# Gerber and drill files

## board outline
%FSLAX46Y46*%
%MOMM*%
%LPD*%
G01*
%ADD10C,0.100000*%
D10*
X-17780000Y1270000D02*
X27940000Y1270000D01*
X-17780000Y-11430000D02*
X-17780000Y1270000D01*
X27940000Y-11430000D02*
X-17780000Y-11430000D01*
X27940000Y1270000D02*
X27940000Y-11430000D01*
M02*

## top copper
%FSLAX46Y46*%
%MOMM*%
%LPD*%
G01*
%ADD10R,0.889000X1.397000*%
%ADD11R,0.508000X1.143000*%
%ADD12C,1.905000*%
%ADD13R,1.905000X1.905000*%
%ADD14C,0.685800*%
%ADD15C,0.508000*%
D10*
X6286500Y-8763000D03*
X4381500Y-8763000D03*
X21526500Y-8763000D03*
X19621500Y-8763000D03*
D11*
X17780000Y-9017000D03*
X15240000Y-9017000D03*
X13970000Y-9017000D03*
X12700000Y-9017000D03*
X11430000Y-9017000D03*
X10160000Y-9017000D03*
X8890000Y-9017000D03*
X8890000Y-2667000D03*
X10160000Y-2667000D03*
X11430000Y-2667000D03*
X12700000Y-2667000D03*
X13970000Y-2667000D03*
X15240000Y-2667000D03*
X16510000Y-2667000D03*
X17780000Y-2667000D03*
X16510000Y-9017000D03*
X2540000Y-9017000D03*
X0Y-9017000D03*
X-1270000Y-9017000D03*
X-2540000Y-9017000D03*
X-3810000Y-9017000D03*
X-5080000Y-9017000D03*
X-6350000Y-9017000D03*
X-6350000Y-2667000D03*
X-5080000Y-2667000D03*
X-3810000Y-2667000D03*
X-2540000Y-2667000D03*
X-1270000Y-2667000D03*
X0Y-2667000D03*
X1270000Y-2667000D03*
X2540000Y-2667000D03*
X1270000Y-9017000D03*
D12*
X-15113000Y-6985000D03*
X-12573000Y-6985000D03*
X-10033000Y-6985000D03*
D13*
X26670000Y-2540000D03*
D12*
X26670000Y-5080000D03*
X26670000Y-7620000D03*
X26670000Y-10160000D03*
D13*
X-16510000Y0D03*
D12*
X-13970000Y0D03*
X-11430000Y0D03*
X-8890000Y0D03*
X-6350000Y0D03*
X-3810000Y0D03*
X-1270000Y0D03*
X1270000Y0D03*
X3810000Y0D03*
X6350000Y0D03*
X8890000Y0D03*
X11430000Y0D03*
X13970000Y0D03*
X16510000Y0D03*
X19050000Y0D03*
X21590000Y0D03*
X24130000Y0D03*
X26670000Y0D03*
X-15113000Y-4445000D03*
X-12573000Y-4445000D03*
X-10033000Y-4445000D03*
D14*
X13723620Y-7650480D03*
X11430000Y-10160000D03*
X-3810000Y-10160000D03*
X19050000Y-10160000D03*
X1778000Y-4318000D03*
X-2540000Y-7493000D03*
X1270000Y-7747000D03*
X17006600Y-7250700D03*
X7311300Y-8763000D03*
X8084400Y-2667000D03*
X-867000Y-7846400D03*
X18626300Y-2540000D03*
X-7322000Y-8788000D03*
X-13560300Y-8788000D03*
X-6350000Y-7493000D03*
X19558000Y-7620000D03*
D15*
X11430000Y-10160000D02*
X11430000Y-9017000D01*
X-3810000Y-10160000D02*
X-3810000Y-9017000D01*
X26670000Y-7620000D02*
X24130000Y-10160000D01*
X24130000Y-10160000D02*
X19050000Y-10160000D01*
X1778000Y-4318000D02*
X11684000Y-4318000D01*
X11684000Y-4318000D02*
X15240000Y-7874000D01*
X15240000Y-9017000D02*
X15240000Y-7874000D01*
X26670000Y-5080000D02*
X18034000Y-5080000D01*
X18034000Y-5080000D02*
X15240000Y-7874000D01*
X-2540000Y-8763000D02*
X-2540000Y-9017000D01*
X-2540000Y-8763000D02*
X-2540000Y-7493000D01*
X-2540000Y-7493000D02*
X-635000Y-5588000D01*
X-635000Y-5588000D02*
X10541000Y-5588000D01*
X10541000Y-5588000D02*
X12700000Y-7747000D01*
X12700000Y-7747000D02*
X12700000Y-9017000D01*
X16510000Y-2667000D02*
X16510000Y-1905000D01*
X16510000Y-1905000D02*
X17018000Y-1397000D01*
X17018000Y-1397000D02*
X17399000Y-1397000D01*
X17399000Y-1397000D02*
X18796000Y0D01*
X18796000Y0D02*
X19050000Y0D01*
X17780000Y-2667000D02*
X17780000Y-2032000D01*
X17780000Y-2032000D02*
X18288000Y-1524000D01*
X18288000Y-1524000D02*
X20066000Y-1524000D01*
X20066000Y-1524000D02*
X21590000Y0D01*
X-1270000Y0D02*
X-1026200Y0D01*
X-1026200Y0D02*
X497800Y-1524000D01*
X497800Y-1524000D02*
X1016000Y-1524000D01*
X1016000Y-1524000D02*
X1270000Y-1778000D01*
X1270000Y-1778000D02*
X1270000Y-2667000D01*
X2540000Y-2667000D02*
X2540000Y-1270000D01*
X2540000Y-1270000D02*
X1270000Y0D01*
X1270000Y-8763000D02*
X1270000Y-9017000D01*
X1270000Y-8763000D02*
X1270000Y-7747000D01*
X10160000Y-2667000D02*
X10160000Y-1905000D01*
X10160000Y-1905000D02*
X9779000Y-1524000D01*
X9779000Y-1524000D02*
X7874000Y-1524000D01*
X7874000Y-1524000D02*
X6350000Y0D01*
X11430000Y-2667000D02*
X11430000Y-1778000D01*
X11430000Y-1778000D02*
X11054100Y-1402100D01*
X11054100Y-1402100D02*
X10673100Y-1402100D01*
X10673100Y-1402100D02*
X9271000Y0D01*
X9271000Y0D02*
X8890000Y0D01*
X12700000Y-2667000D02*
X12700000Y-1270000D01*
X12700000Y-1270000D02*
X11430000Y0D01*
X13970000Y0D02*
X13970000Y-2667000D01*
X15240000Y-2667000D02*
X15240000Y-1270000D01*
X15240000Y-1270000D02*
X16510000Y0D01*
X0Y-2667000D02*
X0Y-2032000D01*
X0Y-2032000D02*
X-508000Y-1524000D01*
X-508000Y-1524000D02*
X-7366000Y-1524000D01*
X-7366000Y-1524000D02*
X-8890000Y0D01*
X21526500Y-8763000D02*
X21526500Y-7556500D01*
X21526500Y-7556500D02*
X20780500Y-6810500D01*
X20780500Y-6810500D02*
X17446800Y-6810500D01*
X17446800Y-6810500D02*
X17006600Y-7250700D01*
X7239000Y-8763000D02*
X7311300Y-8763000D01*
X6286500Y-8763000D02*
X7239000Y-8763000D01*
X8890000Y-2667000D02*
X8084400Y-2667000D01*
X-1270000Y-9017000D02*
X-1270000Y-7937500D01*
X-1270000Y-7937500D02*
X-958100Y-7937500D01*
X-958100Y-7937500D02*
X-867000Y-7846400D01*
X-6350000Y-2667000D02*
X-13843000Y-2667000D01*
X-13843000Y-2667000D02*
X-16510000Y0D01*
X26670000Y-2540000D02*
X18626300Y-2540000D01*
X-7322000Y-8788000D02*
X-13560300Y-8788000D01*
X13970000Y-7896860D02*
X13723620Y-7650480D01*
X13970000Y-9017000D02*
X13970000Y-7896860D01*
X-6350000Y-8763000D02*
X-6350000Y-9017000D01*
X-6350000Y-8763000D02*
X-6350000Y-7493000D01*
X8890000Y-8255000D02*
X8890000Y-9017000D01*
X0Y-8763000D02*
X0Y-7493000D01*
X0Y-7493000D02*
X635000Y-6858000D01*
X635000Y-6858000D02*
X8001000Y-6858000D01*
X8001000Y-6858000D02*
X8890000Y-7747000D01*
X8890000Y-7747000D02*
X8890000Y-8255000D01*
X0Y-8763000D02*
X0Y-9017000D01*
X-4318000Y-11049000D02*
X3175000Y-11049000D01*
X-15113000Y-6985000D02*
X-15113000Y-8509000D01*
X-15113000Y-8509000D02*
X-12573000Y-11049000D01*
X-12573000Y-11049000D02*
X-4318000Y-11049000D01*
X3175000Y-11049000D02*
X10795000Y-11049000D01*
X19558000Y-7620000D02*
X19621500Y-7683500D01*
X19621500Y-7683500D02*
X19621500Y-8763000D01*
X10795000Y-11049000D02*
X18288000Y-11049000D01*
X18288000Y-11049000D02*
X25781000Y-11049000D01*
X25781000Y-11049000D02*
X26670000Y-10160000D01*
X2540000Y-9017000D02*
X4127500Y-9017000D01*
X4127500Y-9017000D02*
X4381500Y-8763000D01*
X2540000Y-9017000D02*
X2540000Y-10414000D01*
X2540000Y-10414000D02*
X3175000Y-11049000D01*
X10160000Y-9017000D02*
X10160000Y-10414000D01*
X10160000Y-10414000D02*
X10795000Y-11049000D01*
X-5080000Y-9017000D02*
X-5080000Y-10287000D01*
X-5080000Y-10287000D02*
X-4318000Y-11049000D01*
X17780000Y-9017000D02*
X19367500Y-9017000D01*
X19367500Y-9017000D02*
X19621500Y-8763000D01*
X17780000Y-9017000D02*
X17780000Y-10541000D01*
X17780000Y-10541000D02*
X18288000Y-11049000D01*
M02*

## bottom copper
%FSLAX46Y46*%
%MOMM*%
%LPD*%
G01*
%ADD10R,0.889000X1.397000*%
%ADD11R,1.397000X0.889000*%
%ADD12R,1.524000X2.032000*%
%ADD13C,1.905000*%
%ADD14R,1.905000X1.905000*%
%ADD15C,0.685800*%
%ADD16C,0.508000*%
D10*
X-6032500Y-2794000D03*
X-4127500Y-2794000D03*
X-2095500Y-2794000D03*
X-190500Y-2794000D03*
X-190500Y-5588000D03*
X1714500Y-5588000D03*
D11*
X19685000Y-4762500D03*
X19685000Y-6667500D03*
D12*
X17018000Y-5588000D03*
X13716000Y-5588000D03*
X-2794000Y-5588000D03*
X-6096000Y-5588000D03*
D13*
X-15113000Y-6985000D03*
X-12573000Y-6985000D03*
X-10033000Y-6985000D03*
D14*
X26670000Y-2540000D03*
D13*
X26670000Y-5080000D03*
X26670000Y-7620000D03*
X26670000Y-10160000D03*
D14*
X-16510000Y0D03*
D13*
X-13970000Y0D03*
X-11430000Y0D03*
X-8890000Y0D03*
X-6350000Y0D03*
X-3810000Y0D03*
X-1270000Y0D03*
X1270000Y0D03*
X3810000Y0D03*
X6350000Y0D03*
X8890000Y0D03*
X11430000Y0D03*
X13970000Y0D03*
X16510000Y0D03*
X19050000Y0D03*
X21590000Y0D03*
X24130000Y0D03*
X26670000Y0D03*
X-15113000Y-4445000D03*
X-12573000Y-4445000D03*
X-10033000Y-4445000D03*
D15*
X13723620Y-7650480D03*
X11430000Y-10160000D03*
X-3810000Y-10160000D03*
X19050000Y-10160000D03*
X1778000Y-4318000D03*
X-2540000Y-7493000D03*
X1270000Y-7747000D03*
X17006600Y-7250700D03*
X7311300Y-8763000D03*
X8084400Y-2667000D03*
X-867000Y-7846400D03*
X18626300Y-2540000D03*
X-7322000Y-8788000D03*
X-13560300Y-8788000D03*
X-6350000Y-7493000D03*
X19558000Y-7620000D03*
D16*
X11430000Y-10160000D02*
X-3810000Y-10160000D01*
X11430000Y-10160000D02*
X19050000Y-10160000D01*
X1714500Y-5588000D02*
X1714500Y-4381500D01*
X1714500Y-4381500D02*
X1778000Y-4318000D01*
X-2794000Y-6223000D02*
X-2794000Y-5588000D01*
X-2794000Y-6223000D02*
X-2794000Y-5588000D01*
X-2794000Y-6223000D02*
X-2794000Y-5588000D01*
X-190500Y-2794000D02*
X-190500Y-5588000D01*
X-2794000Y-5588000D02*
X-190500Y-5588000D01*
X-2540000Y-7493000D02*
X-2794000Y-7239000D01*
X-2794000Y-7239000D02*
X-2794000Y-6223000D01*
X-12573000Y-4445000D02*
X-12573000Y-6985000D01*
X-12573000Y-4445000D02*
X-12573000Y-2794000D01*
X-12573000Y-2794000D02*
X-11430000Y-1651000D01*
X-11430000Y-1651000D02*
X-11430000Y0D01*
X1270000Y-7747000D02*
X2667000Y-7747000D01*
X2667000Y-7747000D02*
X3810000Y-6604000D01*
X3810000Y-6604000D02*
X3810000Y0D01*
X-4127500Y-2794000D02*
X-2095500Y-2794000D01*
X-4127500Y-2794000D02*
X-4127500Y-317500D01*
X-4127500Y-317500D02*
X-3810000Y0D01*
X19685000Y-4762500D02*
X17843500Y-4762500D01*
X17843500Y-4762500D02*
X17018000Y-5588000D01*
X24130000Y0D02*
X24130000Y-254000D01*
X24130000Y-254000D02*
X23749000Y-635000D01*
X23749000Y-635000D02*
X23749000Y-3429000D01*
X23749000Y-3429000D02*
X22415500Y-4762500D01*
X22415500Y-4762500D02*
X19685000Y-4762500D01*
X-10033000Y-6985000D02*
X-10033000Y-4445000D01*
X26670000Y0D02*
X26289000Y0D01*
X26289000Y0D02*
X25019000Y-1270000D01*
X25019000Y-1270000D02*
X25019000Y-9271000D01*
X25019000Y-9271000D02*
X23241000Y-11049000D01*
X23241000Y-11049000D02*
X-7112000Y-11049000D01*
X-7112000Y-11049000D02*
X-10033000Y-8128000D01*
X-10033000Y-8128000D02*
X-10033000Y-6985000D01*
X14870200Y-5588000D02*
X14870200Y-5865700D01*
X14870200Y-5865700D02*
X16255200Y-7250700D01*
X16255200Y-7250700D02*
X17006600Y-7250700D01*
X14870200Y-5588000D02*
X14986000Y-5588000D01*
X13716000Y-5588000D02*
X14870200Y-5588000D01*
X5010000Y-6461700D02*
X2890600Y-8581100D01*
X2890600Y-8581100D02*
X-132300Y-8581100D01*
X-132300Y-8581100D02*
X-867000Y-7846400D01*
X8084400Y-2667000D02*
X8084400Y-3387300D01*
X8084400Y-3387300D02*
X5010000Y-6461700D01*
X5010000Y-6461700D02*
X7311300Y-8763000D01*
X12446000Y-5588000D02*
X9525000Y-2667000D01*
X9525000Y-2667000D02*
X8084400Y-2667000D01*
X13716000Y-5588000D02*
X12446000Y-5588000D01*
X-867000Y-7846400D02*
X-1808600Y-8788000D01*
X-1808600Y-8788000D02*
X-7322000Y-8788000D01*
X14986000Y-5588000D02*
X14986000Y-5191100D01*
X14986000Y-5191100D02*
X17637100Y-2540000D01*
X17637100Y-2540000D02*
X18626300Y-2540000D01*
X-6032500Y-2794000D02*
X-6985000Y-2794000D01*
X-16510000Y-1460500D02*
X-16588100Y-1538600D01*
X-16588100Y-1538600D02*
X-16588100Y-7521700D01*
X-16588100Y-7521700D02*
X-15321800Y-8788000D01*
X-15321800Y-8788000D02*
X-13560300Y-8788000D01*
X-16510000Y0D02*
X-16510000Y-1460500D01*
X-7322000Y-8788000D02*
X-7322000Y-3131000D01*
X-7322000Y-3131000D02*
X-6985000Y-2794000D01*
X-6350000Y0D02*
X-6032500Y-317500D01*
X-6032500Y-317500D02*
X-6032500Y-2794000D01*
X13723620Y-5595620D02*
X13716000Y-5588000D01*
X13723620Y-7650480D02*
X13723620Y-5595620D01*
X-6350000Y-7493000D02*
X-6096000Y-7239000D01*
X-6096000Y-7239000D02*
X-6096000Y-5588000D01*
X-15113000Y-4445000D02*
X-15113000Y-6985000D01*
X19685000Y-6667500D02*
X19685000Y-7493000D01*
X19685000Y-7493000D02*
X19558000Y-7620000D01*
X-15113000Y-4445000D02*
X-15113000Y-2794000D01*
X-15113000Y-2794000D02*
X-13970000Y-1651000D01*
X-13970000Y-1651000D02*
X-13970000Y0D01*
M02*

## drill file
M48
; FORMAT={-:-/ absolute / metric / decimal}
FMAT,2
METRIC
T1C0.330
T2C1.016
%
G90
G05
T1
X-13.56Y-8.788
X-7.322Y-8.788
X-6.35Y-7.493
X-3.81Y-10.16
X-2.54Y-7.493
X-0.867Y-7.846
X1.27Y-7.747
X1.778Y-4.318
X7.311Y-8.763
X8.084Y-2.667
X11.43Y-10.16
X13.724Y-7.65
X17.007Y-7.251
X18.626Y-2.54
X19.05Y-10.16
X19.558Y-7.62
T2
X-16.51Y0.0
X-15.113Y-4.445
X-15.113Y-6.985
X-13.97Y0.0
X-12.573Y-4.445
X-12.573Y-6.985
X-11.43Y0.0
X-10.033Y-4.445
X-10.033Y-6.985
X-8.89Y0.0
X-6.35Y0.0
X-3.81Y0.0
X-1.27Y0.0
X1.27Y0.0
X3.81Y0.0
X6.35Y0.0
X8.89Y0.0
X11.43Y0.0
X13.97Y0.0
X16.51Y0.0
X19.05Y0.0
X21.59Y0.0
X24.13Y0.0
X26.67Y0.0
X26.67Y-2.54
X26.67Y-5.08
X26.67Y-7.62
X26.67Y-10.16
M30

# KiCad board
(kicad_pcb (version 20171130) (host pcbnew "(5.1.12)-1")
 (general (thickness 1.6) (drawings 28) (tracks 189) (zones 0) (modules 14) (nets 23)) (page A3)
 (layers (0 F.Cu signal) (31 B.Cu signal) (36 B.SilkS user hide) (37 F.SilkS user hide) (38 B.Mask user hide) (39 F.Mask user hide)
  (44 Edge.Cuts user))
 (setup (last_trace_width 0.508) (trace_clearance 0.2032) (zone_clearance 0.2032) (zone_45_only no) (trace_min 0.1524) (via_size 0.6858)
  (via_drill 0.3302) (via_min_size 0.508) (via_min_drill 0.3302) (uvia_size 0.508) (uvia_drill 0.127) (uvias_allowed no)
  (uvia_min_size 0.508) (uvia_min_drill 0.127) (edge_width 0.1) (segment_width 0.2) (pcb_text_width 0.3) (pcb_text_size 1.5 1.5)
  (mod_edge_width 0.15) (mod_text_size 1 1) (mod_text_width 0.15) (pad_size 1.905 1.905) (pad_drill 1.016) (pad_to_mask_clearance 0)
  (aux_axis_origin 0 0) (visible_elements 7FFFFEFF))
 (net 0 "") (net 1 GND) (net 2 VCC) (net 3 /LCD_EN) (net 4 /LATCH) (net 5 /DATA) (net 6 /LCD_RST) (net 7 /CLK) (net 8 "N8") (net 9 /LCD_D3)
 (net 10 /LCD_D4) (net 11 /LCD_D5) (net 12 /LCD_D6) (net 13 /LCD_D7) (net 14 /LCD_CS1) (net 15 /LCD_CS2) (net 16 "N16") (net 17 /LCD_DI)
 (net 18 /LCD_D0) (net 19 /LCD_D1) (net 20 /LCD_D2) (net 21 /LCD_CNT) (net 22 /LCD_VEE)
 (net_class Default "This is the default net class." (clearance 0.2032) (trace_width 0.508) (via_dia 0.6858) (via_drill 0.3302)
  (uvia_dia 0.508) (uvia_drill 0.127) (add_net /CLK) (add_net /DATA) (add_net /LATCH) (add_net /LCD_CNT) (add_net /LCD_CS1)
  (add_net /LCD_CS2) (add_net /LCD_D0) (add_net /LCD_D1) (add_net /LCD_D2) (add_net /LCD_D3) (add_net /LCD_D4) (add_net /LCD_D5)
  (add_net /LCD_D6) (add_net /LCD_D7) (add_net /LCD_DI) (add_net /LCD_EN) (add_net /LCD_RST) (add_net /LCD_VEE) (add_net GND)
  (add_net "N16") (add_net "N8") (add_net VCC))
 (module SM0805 (layer F.Cu) (at 5.334 8.763 180)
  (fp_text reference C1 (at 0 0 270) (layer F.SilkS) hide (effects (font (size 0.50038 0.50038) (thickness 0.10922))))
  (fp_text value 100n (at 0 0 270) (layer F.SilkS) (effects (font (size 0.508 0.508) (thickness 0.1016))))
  (pad 1 smd rect (at -0.9525 0 180) (size 0.889 1.397) (layers F.Cu F.Mask) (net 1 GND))
  (pad 2 smd rect (at 0.9525 0 180) (size 0.889 1.397) (layers F.Cu F.Mask) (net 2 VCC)))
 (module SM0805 (layer F.Cu) (at 20.574 8.763 180)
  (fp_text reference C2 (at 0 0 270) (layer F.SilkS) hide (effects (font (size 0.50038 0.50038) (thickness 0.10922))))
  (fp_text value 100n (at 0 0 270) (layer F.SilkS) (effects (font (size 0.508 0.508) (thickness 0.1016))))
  (pad 1 smd rect (at -0.9525 0 180) (size 0.889 1.397) (layers F.Cu F.Mask) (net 1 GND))
  (pad 2 smd rect (at 0.9525 0 180) (size 0.889 1.397) (layers F.Cu F.Mask) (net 2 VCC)))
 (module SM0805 (layer B.Cu) (at -5.08 2.794)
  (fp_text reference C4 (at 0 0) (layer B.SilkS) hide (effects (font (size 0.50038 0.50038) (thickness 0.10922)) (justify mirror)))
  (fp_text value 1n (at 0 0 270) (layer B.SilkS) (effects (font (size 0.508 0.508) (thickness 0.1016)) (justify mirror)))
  (pad 1 smd rect (at -0.9525 0) (size 0.889 1.397) (layers B.Cu B.Mask) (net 1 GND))
  (pad 2 smd rect (at 0.9525 0) (size 0.889 1.397) (layers B.Cu B.Mask) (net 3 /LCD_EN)))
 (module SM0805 (layer B.Cu) (at -1.143 2.794)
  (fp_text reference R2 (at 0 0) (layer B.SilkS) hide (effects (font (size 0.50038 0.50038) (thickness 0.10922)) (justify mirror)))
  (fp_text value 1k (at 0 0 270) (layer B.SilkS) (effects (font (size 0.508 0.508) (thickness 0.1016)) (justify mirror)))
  (pad 1 smd rect (at -0.9525 0) (size 0.889 1.397) (layers B.Cu B.Mask) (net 3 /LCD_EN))
  (pad 2 smd rect (at 0.9525 0) (size 0.889 1.397) (layers B.Cu B.Mask) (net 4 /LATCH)))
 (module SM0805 (layer B.Cu) (at 0.762 5.588)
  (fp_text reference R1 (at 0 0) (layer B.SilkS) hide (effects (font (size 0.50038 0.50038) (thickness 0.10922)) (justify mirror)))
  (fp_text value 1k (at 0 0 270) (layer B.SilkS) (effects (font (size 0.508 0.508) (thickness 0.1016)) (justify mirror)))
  (pad 1 smd rect (at -0.9525 0) (size 0.889 1.397) (layers B.Cu B.Mask) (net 4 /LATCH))
  (pad 2 smd rect (at 0.9525 0) (size 0.889 1.397) (layers B.Cu B.Mask) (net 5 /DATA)))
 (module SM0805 (layer B.Cu) (at 19.685 5.715 270)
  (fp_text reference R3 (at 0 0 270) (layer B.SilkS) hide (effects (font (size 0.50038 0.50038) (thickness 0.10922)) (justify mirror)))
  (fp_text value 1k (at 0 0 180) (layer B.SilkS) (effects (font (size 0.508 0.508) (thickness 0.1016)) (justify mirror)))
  (pad 1 smd rect (at -0.9525 0 270) (size 0.889 1.397) (layers B.Cu B.Mask) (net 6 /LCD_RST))
  (pad 2 smd rect (at 0.9525 0 270) (size 0.889 1.397) (layers B.Cu B.Mask) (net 2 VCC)))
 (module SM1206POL (layer B.Cu) (at 15.367 5.588 180)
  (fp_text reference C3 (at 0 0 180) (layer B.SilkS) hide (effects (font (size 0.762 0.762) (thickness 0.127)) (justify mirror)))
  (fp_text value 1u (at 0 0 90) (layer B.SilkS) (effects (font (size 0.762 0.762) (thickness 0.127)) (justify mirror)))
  (pad 1 smd rect (at -1.651 0 180) (size 1.524 2.032) (layers B.Cu B.Mask) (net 6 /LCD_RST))
  (pad 2 smd rect (at 1.651 0 180) (size 1.524 2.032) (layers B.Cu B.Mask) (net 1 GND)))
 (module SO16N (layer F.Cu) (at 13.335 5.842 180)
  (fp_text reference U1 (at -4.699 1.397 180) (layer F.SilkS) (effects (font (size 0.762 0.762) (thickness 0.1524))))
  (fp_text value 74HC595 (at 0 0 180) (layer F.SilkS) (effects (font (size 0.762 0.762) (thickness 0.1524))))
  (pad 16 smd rect (at -4.445 -3.175 180) (size 0.508 1.143) (layers F.Cu F.Mask) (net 2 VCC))
  (pad 14 smd rect (at -1.905 -3.175 180) (size 0.508 1.143) (layers F.Cu F.Mask) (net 5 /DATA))
  (pad 13 smd rect (at -0.635 -3.175 180) (size 0.508 1.143) (layers F.Cu F.Mask) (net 1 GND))
  (pad 12 smd rect (at 0.635 -3.175 180) (size 0.508 1.143) (layers F.Cu F.Mask) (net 4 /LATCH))
  (pad 11 smd rect (at 1.905 -3.175 180) (size 0.508 1.143) (layers F.Cu F.Mask) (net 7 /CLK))
  (pad 10 smd rect (at 3.175 -3.175 180) (size 0.508 1.143) (layers F.Cu F.Mask) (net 2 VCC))
  (pad 9 smd rect (at 4.445 -3.175 180) (size 0.508 1.143) (layers F.Cu F.Mask) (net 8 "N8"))
  (pad 8 smd rect (at 4.445 3.175 180) (size 0.508 1.143) (layers F.Cu F.Mask) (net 1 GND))
  (pad 7 smd rect (at 3.175 3.175 180) (size 0.508 1.143) (layers F.Cu F.Mask) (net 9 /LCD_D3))
  (pad 6 smd rect (at 1.905 3.175 180) (size 0.508 1.143) (layers F.Cu F.Mask) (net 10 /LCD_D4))
  (pad 5 smd rect (at 0.635 3.175 180) (size 0.508 1.143) (layers F.Cu F.Mask) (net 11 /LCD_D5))
  (pad 4 smd rect (at -0.635 3.175 180) (size 0.508 1.143) (layers F.Cu F.Mask) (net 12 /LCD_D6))
  (pad 3 smd rect (at -1.905 3.175 180) (size 0.508 1.143) (layers F.Cu F.Mask) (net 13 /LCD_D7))
  (pad 2 smd rect (at -3.175 3.175 180) (size 0.508 1.143) (layers F.Cu F.Mask) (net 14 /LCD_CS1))
  (pad 1 smd rect (at -4.445 3.175 180) (size 0.508 1.143) (layers F.Cu F.Mask) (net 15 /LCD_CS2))
  (pad 15 smd rect (at -3.175 -3.175 180) (size 0.508 1.143) (layers F.Cu F.Mask)))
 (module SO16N (layer F.Cu) (at -1.905 5.842 180)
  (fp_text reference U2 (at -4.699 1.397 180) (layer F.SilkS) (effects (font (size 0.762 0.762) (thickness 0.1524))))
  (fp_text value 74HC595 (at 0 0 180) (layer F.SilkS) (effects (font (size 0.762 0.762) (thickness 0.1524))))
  (pad 16 smd rect (at -4.445 -3.175 180) (size 0.508 1.143) (layers F.Cu F.Mask) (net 2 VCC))
  (pad 14 smd rect (at -1.905 -3.175 180) (size 0.508 1.143) (layers F.Cu F.Mask) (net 8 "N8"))
  (pad 13 smd rect (at -0.635 -3.175 180) (size 0.508 1.143) (layers F.Cu F.Mask) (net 1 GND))
  (pad 12 smd rect (at 0.635 -3.175 180) (size 0.508 1.143) (layers F.Cu F.Mask) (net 4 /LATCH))
  (pad 11 smd rect (at 1.905 -3.175 180) (size 0.508 1.143) (layers F.Cu F.Mask) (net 7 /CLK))
  (pad 10 smd rect (at 3.175 -3.175 180) (size 0.508 1.143) (layers F.Cu F.Mask) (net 2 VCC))
  (pad 9 smd rect (at 4.445 -3.175 180) (size 0.508 1.143) (layers F.Cu F.Mask) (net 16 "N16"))
  (pad 8 smd rect (at 4.445 3.175 180) (size 0.508 1.143) (layers F.Cu F.Mask) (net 1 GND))
  (pad 7 smd rect (at 3.175 3.175 180) (size 0.508 1.143) (layers F.Cu F.Mask))
  (pad 6 smd rect (at 1.905 3.175 180) (size 0.508 1.143) (layers F.Cu F.Mask))
  (pad 5 smd rect (at 0.635 3.175 180) (size 0.508 1.143) (layers F.Cu F.Mask))
  (pad 4 smd rect (at -0.635 3.175 180) (size 0.508 1.143) (layers F.Cu F.Mask))
  (pad 3 smd rect (at -1.905 3.175 180) (size 0.508 1.143) (layers F.Cu F.Mask) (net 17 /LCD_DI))
  (pad 2 smd rect (at -3.175 3.175 180) (size 0.508 1.143) (layers F.Cu F.Mask) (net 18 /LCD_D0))
  (pad 1 smd rect (at -4.445 3.175 180) (size 0.508 1.143) (layers F.Cu F.Mask) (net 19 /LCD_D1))
  (pad 15 smd rect (at -3.175 -3.175 180) (size 0.508 1.143) (layers F.Cu F.Mask) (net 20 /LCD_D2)))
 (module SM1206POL (layer B.Cu) (at -4.445 5.588 180)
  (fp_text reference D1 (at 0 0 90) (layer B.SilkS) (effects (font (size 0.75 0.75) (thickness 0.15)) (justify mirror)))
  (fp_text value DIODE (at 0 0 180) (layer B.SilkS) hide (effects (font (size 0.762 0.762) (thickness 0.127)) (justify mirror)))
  (pad 1 smd rect (at -1.651 0 180) (size 1.524 2.032) (layers B.Cu B.Mask) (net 4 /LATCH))
  (pad 2 smd rect (at 1.651 0 180) (size 1.524 2.032) (layers B.Cu B.Mask) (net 16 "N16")))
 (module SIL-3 (layer B.Cu) (at -12.573 6.985)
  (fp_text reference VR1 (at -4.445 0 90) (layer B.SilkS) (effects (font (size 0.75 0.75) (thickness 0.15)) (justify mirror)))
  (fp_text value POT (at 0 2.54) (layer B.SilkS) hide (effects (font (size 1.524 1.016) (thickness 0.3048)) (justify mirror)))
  (pad 1 thru_hole circle (at -2.54 0) (size 1.905 1.905) (drill 1.016) (layers *.Cu *.Mask B.SilkS) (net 2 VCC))
  (pad 2 thru_hole circle (at 0 0) (size 1.905 1.905) (drill 1.016) (layers *.Cu *.Mask B.SilkS) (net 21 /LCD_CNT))
  (pad 3 thru_hole circle (at 2.54 0) (size 1.905 1.905) (drill 1.016) (layers *.Cu *.Mask B.SilkS) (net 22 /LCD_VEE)))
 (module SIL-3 (layer B.Cu) (at 26.67 5.08 270)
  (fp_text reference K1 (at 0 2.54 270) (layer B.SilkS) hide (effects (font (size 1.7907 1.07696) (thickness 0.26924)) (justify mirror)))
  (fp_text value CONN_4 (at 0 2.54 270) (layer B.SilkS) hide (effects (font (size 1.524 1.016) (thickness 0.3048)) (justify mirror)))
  (pad 1 thru_hole rect (at -2.54 0 270) (size 1.905 1.905) (drill 1.016) (layers *.Cu *.Mask B.SilkS) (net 1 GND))
  (pad 2 thru_hole circle (at 0 0 270) (size 1.905 1.905) (drill 1.016) (layers *.Cu *.Mask B.SilkS) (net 5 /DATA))
  (pad 3 thru_hole circle (at 2.54 0 270) (size 1.905 1.905) (drill 1.016) (layers *.Cu *.Mask B.SilkS) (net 7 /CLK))
  (pad 4 thru_hole circle (at 5.08 0 270) (size 1.905 1.905) (drill 1.016) (layers *.Cu *.Mask B.SilkS) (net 2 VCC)))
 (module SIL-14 (layer F.Cu) (at 0 0)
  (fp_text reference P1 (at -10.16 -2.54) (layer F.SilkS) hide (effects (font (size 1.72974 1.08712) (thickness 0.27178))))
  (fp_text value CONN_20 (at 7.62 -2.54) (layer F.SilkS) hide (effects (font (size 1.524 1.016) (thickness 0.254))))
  (pad 1 thru_hole rect (at -16.51 0) (size 1.905 1.905) (drill 1.016) (layers *.Cu *.Mask F.SilkS) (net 1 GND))
  (pad 2 thru_hole circle (at -13.97 0) (size 1.905 1.905) (drill 1.016) (layers *.Cu *.Mask F.SilkS) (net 2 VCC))
  (pad 3 thru_hole circle (at -11.43 0) (size 1.905 1.905) (drill 1.016) (layers *.Cu *.Mask F.SilkS) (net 21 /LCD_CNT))
  (pad 4 thru_hole circle (at -8.89 0) (size 1.905 1.905) (drill 1.016) (layers *.Cu *.Mask F.SilkS) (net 17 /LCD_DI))
  (pad 5 thru_hole circle (at -6.35 0) (size 1.905 1.905) (drill 1.016) (layers *.Cu *.Mask F.SilkS) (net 1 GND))
  (pad 6 thru_hole circle (at -3.81 0) (size 1.905 1.905) (drill 1.016) (layers *.Cu *.Mask F.SilkS) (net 3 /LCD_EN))
  (pad 7 thru_hole circle (at -1.27 0) (size 1.905 1.905) (drill 1.016) (layers *.Cu *.Mask F.SilkS) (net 18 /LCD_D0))
  (pad 8 thru_hole circle (at 1.27 0) (size 1.905 1.905) (drill 1.016) (layers *.Cu *.Mask F.SilkS) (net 19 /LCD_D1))
  (pad 9 thru_hole circle (at 3.81 0) (size 1.905 1.905) (drill 1.016) (layers *.Cu *.Mask F.SilkS) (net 20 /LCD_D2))
  (pad 10 thru_hole circle (at 6.35 0) (size 1.905 1.905) (drill 1.016) (layers *.Cu *.Mask F.SilkS) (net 9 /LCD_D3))
  (pad 11 thru_hole circle (at 8.89 0) (size 1.905 1.905) (drill 1.016) (layers *.Cu *.Mask F.SilkS) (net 10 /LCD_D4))
  (pad 12 thru_hole circle (at 11.43 0) (size 1.905 1.905) (drill 1.016) (layers *.Cu *.Mask F.SilkS) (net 11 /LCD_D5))
  (pad 13 thru_hole circle (at 13.97 0) (size 1.905 1.905) (drill 1.016) (layers *.Cu *.Mask F.SilkS) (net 12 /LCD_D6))
  (pad 14 thru_hole circle (at 16.51 0) (size 1.905 1.905) (drill 1.016) (layers *.Cu *.Mask F.SilkS) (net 13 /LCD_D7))
  (pad 15 thru_hole circle (at 19.05 0) (size 1.905 1.905) (drill 1.016) (layers *.Cu *.Mask F.SilkS) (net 14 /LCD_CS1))
  (pad 16 thru_hole circle (at 21.59 0) (size 1.905 1.905) (drill 1.016) (layers *.Cu *.Mask F.SilkS) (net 15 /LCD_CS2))
  (pad 17 thru_hole circle (at 24.13 0) (size 1.905 1.905) (drill 1.016) (layers *.Cu *.Mask F.SilkS) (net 6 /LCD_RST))
  (pad 18 thru_hole circle (at 26.67 0) (size 1.905 1.905) (drill 1.016) (layers *.Cu *.Mask F.SilkS) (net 22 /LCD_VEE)))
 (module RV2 (layer B.Cu) (at -12.573 5.715) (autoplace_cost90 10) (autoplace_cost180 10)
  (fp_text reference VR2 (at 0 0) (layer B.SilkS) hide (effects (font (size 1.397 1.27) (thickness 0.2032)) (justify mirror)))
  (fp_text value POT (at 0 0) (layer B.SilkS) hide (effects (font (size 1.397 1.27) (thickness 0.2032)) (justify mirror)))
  (pad 1 thru_hole circle (at -2.54 -1.27) (size 1.905 1.905) (drill 1.016) (layers *.Cu *.Mask B.SilkS) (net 2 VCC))
  (pad 2 thru_hole circle (at 0 -1.27) (size 1.905 1.905) (drill 1.016) (layers *.Cu *.Mask B.SilkS) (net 21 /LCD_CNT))
  (pad 3 thru_hole circle (at 2.54 -1.27) (size 1.905 1.905) (drill 1.016) (layers *.Cu *.Mask B.SilkS) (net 22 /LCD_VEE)))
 (gr_line (start -17.78 -1.27) (end 27.94 -1.27) (angle 90) (layer Edge.Cuts) (width 0.1))
 (gr_line (start -17.78 11.43) (end -17.78 -1.27) (angle 90) (layer Edge.Cuts) (width 0.1))
 (gr_line (start 27.94 11.43) (end -17.78 11.43) (angle 90) (layer Edge.Cuts) (width 0.1))
 (gr_line (start 27.94 -1.27) (end 27.94 11.43) (angle 90) (layer Edge.Cuts) (width 0.1))
 (via (at 13.72362 7.65048) (size 0.6858) (drill 0.3302) (layers F.Cu B.Cu) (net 1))
 (segment (start 11.43 10.16) (end 11.43 9.017) (width 0.508) (layer F.Cu) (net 7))
 (segment (start -3.81 10.16) (end -3.81 9.017) (width 0.508) (layer F.Cu) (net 7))
 (segment (start 11.43 10.16) (end -3.81 10.16) (width 0.508) (layer B.Cu) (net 7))
 (segment (start 26.67 7.62) (end 24.13 10.16) (width 0.508) (layer F.Cu) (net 7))
 (segment (start 24.13 10.16) (end 19.05 10.16) (width 0.508) (layer F.Cu) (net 7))
 (segment (start 11.43 10.16) (end 19.05 10.16) (width 0.508) (layer B.Cu) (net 7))
 (via (at 11.43 10.16) (size 0.6858) (layers F.Cu B.Cu) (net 7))
 (via (at -3.81 10.16) (size 0.6858) (layers F.Cu B.Cu) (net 7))
 (via (at 19.05 10.16) (size 0.6858) (layers F.Cu B.Cu) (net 7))
 (segment (start 1.7145 5.588) (end 1.7145 4.3815) (width 0.508) (layer B.Cu) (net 5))
 (segment (start 1.7145 4.3815) (end 1.778 4.318) (width 0.508) (layer B.Cu) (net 5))
 (segment (start 1.778 4.318) (end 11.684 4.318) (width 0.508) (layer F.Cu) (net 5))
 (segment (start 11.684 4.318) (end 15.24 7.874) (width 0.508) (layer F.Cu) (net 5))
 (segment (start 15.24 9.017) (end 15.24 7.874) (width 0.508) (layer F.Cu) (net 5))
 (segment (start 26.67 5.08) (end 18.034 5.08) (width 0.508) (layer F.Cu) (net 5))
 (segment (start 18.034 5.08) (end 15.24 7.874) (width 0.508) (layer F.Cu) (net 5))
 (via (at 1.778 4.318) (size 0.6858) (layers F.Cu B.Cu) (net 5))
 (segment (start -2.54 8.763) (end -2.54 9.017) (width 0.508) (layer F.Cu) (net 4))
 (segment (start -2.54 8.763) (end -2.54 7.493) (width 0.508) (layer F.Cu) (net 4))
 (segment (start -2.794 6.223) (end -2.794 5.588) (width 0.508) (layer B.Cu) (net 4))
 (segment (start -2.794 6.223) (end -2.794 5.588) (width 0.508) (layer B.Cu) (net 4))
 (segment (start -2.794 6.223) (end -2.794 5.588) (width 0.508) (layer B.Cu) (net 4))
 (segment (start -2.54 7.493) (end -0.635 5.588) (width 0.508) (layer F.Cu) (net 4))
 (segment (start -0.635 5.588) (end 10.541 5.588) (width 0.508) (layer F.Cu) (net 4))
 (segment (start 10.541 5.588) (end 12.7 7.747) (width 0.508) (layer F.Cu) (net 4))
 (segment (start 12.7 7.747) (end 12.7 9.017) (width 0.508) (layer F.Cu) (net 4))
 (segment (start -0.1905 2.794) (end -0.1905 5.588) (width 0.508) (layer B.Cu) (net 4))
 (segment (start -2.794 5.588) (end -0.1905 5.588) (width 0.508) (layer B.Cu) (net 4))
 (segment (start -2.54 7.493) (end -2.794 7.239) (width 0.508) (layer B.Cu) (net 4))
 (segment (start -2.794 7.239) (end -2.794 6.223) (width 0.508) (layer B.Cu) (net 4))
 (via (at -2.54 7.493) (size 0.6858) (layers F.Cu B.Cu) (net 4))
 (segment (start -12.573 4.445) (end -12.573 6.985) (width 0.508) (layer B.Cu) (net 21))
 (segment (start -12.573 4.445) (end -12.573 2.794) (width 0.508) (layer B.Cu) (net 21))
 (segment (start -12.573 2.794) (end -11.43 1.651) (width 0.508) (layer B.Cu) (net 21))
 (segment (start -11.43 1.651) (end -11.43 0) (width 0.508) (layer B.Cu) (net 21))
 (segment (start 16.51 2.667) (end 16.51 1.905) (width 0.508) (layer F.Cu) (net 14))
 (segment (start 16.51 1.905) (end 17.018 1.397) (width 0.508) (layer F.Cu) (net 14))
 (segment (start 17.018 1.397) (end 17.399 1.397) (width 0.508) (layer F.Cu) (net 14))
 (segment (start 17.399 1.397) (end 18.796 0) (width 0.508) (layer F.Cu) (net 14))
 (segment (start 18.796 0) (end 19.05 0) (width 0.508) (layer F.Cu) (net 14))
 (segment (start 17.78 2.667) (end 17.78 2.032) (width 0.508) (layer F.Cu) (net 15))
 (segment (start 17.78 2.032) (end 18.288 1.524) (width 0.508) (layer F.Cu) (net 15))
 (segment (start 18.288 1.524) (end 20.066 1.524) (width 0.508) (layer F.Cu) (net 15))
 (segment (start 20.066 1.524) (end 21.59 0) (width 0.508) (layer F.Cu) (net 15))
 (segment (start -1.27 0) (end -1.0262 0) (width 0.508) (layer F.Cu) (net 18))
 (segment (start -1.0262 0) (end 0.4978 1.524) (width 0.508) (layer F.Cu) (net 18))
 (segment (start 0.4978 1.524) (end 1.016 1.524) (width 0.508) (layer F.Cu) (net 18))
 (segment (start 1.016 1.524) (end 1.27 1.778) (width 0.508) (layer F.Cu) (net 18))
 (segment (start 1.27 1.778) (end 1.27 2.667) (width 0.508) (layer F.Cu) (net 18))
 (segment (start 2.54 2.667) (end 2.54 1.27) (width 0.508) (layer F.Cu) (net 19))
 (segment (start 2.54 1.27) (end 1.27 0) (width 0.508) (layer F.Cu) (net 19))
 (segment (start 1.27 8.763) (end 1.27 9.017) (width 0.508) (layer F.Cu) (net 20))
 (segment (start 1.27 8.763) (end 1.27 7.747) (width 0.508) (layer F.Cu) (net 20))
 (segment (start 1.27 7.747) (end 2.667 7.747) (width 0.508) (layer B.Cu) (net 20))
 (segment (start 2.667 7.747) (end 3.81 6.604) (width 0.508) (layer B.Cu) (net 20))
 (segment (start 3.81 6.604) (end 3.81 0) (width 0.508) (layer B.Cu) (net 20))
 (via (at 1.27 7.747) (size 0.6858) (layers F.Cu B.Cu) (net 20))
 (segment (start 10.16 2.667) (end 10.16 1.905) (width 0.508) (layer F.Cu) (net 9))
 (segment (start 10.16 1.905) (end 9.779 1.524) (width 0.508) (layer F.Cu) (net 9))
 (segment (start 9.779 1.524) (end 7.874 1.524) (width 0.508) (layer F.Cu) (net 9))
 (segment (start 7.874 1.524) (end 6.35 0) (width 0.508) (layer F.Cu) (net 9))
 (segment (start 11.43 2.667) (end 11.43 1.778) (width 0.508) (layer F.Cu) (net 10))
 (segment (start 11.43 1.778) (end 11.0541 1.4021) (width 0.508) (layer F.Cu) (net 10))
 (segment (start 11.0541 1.4021) (end 10.6731 1.4021) (width 0.508) (layer F.Cu) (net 10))
 (segment (start 10.6731 1.4021) (end 9.271 0) (width 0.508) (layer F.Cu) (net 10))
 (segment (start 9.271 0) (end 8.89 0) (width 0.508) (layer F.Cu) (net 10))
 (segment (start 12.7 2.667) (end 12.7 1.27) (width 0.508) (layer F.Cu) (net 11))
 (segment (start 12.7 1.27) (end 11.43 0) (width 0.508) (layer F.Cu) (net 11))
 (segment (start 13.97 0) (end 13.97 2.667) (width 0.508) (layer F.Cu) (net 12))
 (segment (start 15.24 2.667) (end 15.24 1.27) (width 0.508) (layer F.Cu) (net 13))
 (segment (start 15.24 1.27) (end 16.51 0) (width 0.508) (layer F.Cu) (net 13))
 (segment (start 0 2.667) (end 0 2.032) (width 0.508) (layer F.Cu) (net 17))
 (segment (start 0 2.032) (end -0.508 1.524) (width 0.508) (layer F.Cu) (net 17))
 (segment (start -0.508 1.524) (end -7.366 1.524) (width 0.508) (layer F.Cu) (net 17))
 (segment (start -7.366 1.524) (end -8.89 0) (width 0.508) (layer F.Cu) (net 17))
 (segment (start -4.1275 2.794) (end -2.0955 2.794) (width 0.508) (layer B.Cu) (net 3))
 (segment (start -4.1275 2.794) (end -4.1275 0.3175) (width 0.508) (layer B.Cu) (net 3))
 (segment (start -4.1275 0.3175) (end -3.81 0) (width 0.508) (layer B.Cu) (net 3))
 (segment (start 19.685 4.7625) (end 17.8435 4.7625) (width 0.508) (layer B.Cu) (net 6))
 (segment (start 17.8435 4.7625) (end 17.018 5.588) (width 0.508) (layer B.Cu) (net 6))
 (segment (start 24.13 0) (end 24.13 0.254) (width 0.508) (layer B.Cu) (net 6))
 (segment (start 24.13 0.254) (end 23.749 0.635) (width 0.508) (layer B.Cu) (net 6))
 (segment (start 23.749 0.635) (end 23.749 3.429) (width 0.508) (layer B.Cu) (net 6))
 (segment (start 23.749 3.429) (end 22.4155 4.7625) (width 0.508) (layer B.Cu) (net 6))
 (segment (start 22.4155 4.7625) (end 19.685 4.7625) (width 0.508) (layer B.Cu) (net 6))
 (segment (start -10.033 6.985) (end -10.033 4.445) (width 0.508) (layer B.Cu) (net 22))
 (segment (start 26.67 0) (end 26.289 0) (width 0.508) (layer B.Cu) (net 22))
 (segment (start 26.289 0) (end 25.019 1.27) (width 0.508) (layer B.Cu) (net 22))
 (segment (start 25.019 1.27) (end 25.019 9.271) (width 0.508) (layer B.Cu) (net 22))
 (segment (start 25.019 9.271) (end 23.241 11.049) (width 0.508) (layer B.Cu) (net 22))
 (segment (start 23.241 11.049) (end -7.112 11.049) (width 0.508) (layer B.Cu) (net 22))
 (segment (start -7.112 11.049) (end -10.033 8.128) (width 0.508) (layer B.Cu) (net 22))
 (segment (start -10.033 8.128) (end -10.033 6.985) (width 0.508) (layer B.Cu) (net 22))
 (segment (start 21.5265 8.763) (end 21.5265 7.5565) (width 0.508) (layer F.Cu) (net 1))
 (segment (start 21.5265 7.5565) (end 20.7805 6.8105) (width 0.508) (layer F.Cu) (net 1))
 (segment (start 20.7805 6.8105) (end 17.4468 6.8105) (width 0.508) (layer F.Cu) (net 1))
 (segment (start 17.4468 6.8105) (end 17.0066 7.2507) (width 0.508) (layer F.Cu) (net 1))
 (segment (start 14.8702 5.588) (end 14.8702 5.8657) (width 0.508) (layer B.Cu) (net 1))
 (segment (start 14.8702 5.8657) (end 16.2552 7.2507) (width 0.508) (layer B.Cu) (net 1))
 (segment (start 16.2552 7.2507) (end 17.0066 7.2507) (width 0.508) (layer B.Cu) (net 1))
 (segment (start 14.8702 5.588) (end 14.986 5.588) (width 0.508) (layer B.Cu) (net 1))
 (segment (start 13.716 5.588) (end 14.8702 5.588) (width 0.508) (layer B.Cu) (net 1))
 (segment (start 5.01 6.4617) (end 2.8906 8.5811) (width 0.508) (layer B.Cu) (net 1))
 (segment (start 2.8906 8.5811) (end -0.1323 8.5811) (width 0.508) (layer B.Cu) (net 1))
 (segment (start -0.1323 8.5811) (end -0.867 7.8464) (width 0.508) (layer B.Cu) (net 1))
 (segment (start 8.0844 2.667) (end 8.0844 3.3873) (width 0.508) (layer B.Cu) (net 1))
 (segment (start 8.0844 3.3873) (end 5.01 6.4617) (width 0.508) (layer B.Cu) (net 1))
 (segment (start 5.01 6.4617) (end 7.3113 8.763) (width 0.508) (layer B.Cu) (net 1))
 (segment (start 7.239 8.763) (end 7.3113 8.763) (width 0.508) (layer F.Cu) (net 1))
 (segment (start 6.2865 8.763) (end 7.239 8.763) (width 0.508) (layer F.Cu) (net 1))
 (segment (start 12.446 5.588) (end 9.525 2.667) (width 0.508) (layer B.Cu) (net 1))
 (segment (start 9.525 2.667) (end 8.0844 2.667) (width 0.508) (layer B.Cu) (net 1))
 (segment (start 8.89 2.667) (end 8.0844 2.667) (width 0.508) (layer F.Cu) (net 1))
 (segment (start 13.716 5.588) (end 12.446 5.588) (width 0.508) (layer B.Cu) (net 1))
 (segment (start -1.27 9.017) (end -1.27 7.9375) (width 0.508) (layer F.Cu) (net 1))
 (segment (start -0.867 7.8464) (end -1.8086 8.788) (width 0.508) (layer B.Cu) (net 1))
 (segment (start -1.8086 8.788) (end -7.322 8.788) (width 0.508) (layer B.Cu) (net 1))
 (segment (start -1.27 7.9375) (end -0.9581 7.9375) (width 0.508) (layer F.Cu) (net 1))
 (segment (start -0.9581 7.9375) (end -0.867 7.8464) (width 0.508) (layer F.Cu) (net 1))
 (segment (start -6.35 2.667) (end -13.843 2.667) (width 0.508) (layer F.Cu) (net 1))
 (segment (start -13.843 2.667) (end -16.51 0) (width 0.508) (layer F.Cu) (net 1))
 (segment (start 26.67 2.54) (end 18.6263 2.54) (width 0.508) (layer F.Cu) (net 1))
 (segment (start 14.986 5.588) (end 14.986 5.1911) (width 0.508) (layer B.Cu) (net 1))
 (segment (start 14.986 5.1911) (end 17.6371 2.54) (width 0.508) (layer B.Cu) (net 1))
 (segment (start 17.6371 2.54) (end 18.6263 2.54) (width 0.508) (layer B.Cu) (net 1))
 (segment (start -6.0325 2.794) (end -6.985 2.794) (width 0.508) (layer B.Cu) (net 1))
 (segment (start -7.322 8.788) (end -13.5603 8.788) (width 0.508) (layer F.Cu) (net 1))
 (segment (start -16.51 1.4605) (end -16.5881 1.5386) (width 0.508) (layer B.Cu) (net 1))
 (segment (start -16.5881 1.5386) (end -16.5881 7.5217) (width 0.508) (layer B.Cu) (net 1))
 (segment (start -16.5881 7.5217) (end -15.3218 8.788) (width 0.508) (layer B.Cu) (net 1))
 (segment (start -15.3218 8.788) (end -13.5603 8.788) (width 0.508) (layer B.Cu) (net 1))
 (segment (start -16.51 0) (end -16.51 1.4605) (width 0.508) (layer B.Cu) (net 1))
 (segment (start -7.322 8.788) (end -7.322 3.131) (width 0.508) (layer B.Cu) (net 1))
 (segment (start -7.322 3.131) (end -6.985 2.794) (width 0.508) (layer B.Cu) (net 1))
 (segment (start -6.35 0) (end -6.0325 0.3175) (width 0.508) (layer B.Cu) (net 1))
 (segment (start -6.0325 0.3175) (end -6.0325 2.794) (width 0.508) (layer B.Cu) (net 1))
 (via (at 17.0066 7.2507) (size 0.6858) (layers F.Cu B.Cu) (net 1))
 (via (at 7.3113 8.763) (size 0.6858) (layers F.Cu B.Cu) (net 1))
 (via (at 8.0844 2.667) (size 0.6858) (layers F.Cu B.Cu) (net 1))
 (via (at -0.867 7.8464) (size 0.6858) (layers F.Cu B.Cu) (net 1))
 (via (at 18.6263 2.54) (size 0.6858) (layers F.Cu B.Cu) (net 1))
 (via (at -7.322 8.788) (size 0.6858) (layers F.Cu B.Cu) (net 1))
 (via (at -13.5603 8.788) (size 0.6858) (layers F.Cu B.Cu) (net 1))
 (segment (start 13.97 7.89686) (end 13.72362 7.65048) (width 0.508) (layer F.Cu) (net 1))
 (segment (start 13.97 9.017) (end 13.97 7.89686) (width 0.508) (layer F.Cu) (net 1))
 (segment (start 13.72362 5.59562) (end 13.716 5.588) (width 0.508) (layer B.Cu) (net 1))
 (segment (start 13.72362 7.65048) (end 13.72362 5.59562) (width 0.508) (layer B.Cu) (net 1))
 (segment (start -6.35 8.763) (end -6.35 9.017) (width 0.508) (layer F.Cu) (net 16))
 (segment (start -6.35 8.763) (end -6.35 7.493) (width 0.508) (layer F.Cu) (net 16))
 (segment (start -6.35 7.493) (end -6.096 7.239) (width 0.508) (layer B.Cu) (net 16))
 (segment (start -6.096 7.239) (end -6.096 5.588) (width 0.508) (layer B.Cu) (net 16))
 (via (at -6.35 7.493) (size 0.6858) (layers F.Cu B.Cu) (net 16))
 (segment (start 8.89 8.255) (end 8.89 9.017) (width 0.508) (layer F.Cu) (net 8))
 (segment (start 0 8.763) (end 0 7.493) (width 0.508) (layer F.Cu) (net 8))
 (segment (start 0 7.493) (end 0.635 6.858) (width 0.508) (layer F.Cu) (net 8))
 (segment (start 0.635 6.858) (end 8.001 6.858) (width 0.508) (layer F.Cu) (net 8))
 (segment (start 8.001 6.858) (end 8.89 7.747) (width 0.508) (layer F.Cu) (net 8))
 (segment (start 8.89 7.747) (end 8.89 8.255) (width 0.508) (layer F.Cu) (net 8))
 (segment (start 0 8.763) (end 0 9.017) (width 0.508) (layer F.Cu) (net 8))
 (segment (start -4.318 11.049) (end 3.175 11.049) (width 0.508) (layer F.Cu) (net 2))
 (segment (start -15.113 6.985) (end -15.113 8.509) (width 0.508) (layer F.Cu) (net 2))
 (segment (start -15.113 8.509) (end -12.573 11.049) (width 0.508) (layer F.Cu) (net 2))
 (segment (start -12.573 11.049) (end -4.318 11.049) (width 0.508) (layer F.Cu) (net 2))
 (segment (start 3.175 11.049) (end 10.795 11.049) (width 0.508) (layer F.Cu) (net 2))
 (segment (start -15.113 4.445) (end -15.113 6.985) (width 0.508) (layer B.Cu) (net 2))
 (segment (start 19.558 7.62) (end 19.6215 7.6835) (width 0.508) (layer F.Cu) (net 2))
 (segment (start 19.6215 7.6835) (end 19.6215 8.763) (width 0.508) (layer F.Cu) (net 2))
 (segment (start 19.685 6.6675) (end 19.685 7.493) (width 0.508) (layer B.Cu) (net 2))
 (segment (start 19.685 7.493) (end 19.558 7.62) (width 0.508) (layer B.Cu) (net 2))
 (segment (start 10.795 11.049) (end 18.288 11.049) (width 0.508) (layer F.Cu) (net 2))
 (segment (start 18.288 11.049) (end 25.781 11.049) (width 0.508) (layer F.Cu) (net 2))
 (segment (start 25.781 11.049) (end 26.67 10.16) (width 0.508) (layer F.Cu) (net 2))
 (segment (start -15.113 4.445) (end -15.113 2.794) (width 0.508) (layer B.Cu) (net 2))
 (segment (start -15.113 2.794) (end -13.97 1.651) (width 0.508) (layer B.Cu) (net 2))
 (segment (start -13.97 1.651) (end -13.97 0) (width 0.508) (layer B.Cu) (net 2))
 (segment (start 2.54 9.017) (end 4.1275 9.017) (width 0.508) (layer F.Cu) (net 2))
 (segment (start 4.1275 9.017) (end 4.3815 8.763) (width 0.508) (layer F.Cu) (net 2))
 (segment (start 2.54 9.017) (end 2.54 10.414) (width 0.508) (layer F.Cu) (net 2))
 (segment (start 2.54 10.414) (end 3.175 11.049) (width 0.508) (layer F.Cu) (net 2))
 (segment (start 10.16 9.017) (end 10.16 10.414) (width 0.508) (layer F.Cu) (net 2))
 (segment (start 10.16 10.414) (end 10.795 11.049) (width 0.508) (layer F.Cu) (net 2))
 (segment (start -5.08 9.017) (end -5.08 10.287) (width 0.508) (layer F.Cu) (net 2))
 (segment (start -5.08 10.287) (end -4.318 11.049) (width 0.508) (layer F.Cu) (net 2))
 (segment (start 17.78 9.017) (end 19.3675 9.017) (width 0.508) (layer F.Cu) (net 2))
 (segment (start 19.3675 9.017) (end 19.6215 8.763) (width 0.508) (layer F.Cu) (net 2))
 (segment (start 17.78 9.017) (end 17.78 10.541) (width 0.508) (layer F.Cu) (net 2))
 (segment (start 17.78 10.541) (end 18.288 11.049) (width 0.508) (layer F.Cu) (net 2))
 (via (at 19.558 7.62) (size 0.6858) (layers F.Cu B.Cu) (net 2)))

